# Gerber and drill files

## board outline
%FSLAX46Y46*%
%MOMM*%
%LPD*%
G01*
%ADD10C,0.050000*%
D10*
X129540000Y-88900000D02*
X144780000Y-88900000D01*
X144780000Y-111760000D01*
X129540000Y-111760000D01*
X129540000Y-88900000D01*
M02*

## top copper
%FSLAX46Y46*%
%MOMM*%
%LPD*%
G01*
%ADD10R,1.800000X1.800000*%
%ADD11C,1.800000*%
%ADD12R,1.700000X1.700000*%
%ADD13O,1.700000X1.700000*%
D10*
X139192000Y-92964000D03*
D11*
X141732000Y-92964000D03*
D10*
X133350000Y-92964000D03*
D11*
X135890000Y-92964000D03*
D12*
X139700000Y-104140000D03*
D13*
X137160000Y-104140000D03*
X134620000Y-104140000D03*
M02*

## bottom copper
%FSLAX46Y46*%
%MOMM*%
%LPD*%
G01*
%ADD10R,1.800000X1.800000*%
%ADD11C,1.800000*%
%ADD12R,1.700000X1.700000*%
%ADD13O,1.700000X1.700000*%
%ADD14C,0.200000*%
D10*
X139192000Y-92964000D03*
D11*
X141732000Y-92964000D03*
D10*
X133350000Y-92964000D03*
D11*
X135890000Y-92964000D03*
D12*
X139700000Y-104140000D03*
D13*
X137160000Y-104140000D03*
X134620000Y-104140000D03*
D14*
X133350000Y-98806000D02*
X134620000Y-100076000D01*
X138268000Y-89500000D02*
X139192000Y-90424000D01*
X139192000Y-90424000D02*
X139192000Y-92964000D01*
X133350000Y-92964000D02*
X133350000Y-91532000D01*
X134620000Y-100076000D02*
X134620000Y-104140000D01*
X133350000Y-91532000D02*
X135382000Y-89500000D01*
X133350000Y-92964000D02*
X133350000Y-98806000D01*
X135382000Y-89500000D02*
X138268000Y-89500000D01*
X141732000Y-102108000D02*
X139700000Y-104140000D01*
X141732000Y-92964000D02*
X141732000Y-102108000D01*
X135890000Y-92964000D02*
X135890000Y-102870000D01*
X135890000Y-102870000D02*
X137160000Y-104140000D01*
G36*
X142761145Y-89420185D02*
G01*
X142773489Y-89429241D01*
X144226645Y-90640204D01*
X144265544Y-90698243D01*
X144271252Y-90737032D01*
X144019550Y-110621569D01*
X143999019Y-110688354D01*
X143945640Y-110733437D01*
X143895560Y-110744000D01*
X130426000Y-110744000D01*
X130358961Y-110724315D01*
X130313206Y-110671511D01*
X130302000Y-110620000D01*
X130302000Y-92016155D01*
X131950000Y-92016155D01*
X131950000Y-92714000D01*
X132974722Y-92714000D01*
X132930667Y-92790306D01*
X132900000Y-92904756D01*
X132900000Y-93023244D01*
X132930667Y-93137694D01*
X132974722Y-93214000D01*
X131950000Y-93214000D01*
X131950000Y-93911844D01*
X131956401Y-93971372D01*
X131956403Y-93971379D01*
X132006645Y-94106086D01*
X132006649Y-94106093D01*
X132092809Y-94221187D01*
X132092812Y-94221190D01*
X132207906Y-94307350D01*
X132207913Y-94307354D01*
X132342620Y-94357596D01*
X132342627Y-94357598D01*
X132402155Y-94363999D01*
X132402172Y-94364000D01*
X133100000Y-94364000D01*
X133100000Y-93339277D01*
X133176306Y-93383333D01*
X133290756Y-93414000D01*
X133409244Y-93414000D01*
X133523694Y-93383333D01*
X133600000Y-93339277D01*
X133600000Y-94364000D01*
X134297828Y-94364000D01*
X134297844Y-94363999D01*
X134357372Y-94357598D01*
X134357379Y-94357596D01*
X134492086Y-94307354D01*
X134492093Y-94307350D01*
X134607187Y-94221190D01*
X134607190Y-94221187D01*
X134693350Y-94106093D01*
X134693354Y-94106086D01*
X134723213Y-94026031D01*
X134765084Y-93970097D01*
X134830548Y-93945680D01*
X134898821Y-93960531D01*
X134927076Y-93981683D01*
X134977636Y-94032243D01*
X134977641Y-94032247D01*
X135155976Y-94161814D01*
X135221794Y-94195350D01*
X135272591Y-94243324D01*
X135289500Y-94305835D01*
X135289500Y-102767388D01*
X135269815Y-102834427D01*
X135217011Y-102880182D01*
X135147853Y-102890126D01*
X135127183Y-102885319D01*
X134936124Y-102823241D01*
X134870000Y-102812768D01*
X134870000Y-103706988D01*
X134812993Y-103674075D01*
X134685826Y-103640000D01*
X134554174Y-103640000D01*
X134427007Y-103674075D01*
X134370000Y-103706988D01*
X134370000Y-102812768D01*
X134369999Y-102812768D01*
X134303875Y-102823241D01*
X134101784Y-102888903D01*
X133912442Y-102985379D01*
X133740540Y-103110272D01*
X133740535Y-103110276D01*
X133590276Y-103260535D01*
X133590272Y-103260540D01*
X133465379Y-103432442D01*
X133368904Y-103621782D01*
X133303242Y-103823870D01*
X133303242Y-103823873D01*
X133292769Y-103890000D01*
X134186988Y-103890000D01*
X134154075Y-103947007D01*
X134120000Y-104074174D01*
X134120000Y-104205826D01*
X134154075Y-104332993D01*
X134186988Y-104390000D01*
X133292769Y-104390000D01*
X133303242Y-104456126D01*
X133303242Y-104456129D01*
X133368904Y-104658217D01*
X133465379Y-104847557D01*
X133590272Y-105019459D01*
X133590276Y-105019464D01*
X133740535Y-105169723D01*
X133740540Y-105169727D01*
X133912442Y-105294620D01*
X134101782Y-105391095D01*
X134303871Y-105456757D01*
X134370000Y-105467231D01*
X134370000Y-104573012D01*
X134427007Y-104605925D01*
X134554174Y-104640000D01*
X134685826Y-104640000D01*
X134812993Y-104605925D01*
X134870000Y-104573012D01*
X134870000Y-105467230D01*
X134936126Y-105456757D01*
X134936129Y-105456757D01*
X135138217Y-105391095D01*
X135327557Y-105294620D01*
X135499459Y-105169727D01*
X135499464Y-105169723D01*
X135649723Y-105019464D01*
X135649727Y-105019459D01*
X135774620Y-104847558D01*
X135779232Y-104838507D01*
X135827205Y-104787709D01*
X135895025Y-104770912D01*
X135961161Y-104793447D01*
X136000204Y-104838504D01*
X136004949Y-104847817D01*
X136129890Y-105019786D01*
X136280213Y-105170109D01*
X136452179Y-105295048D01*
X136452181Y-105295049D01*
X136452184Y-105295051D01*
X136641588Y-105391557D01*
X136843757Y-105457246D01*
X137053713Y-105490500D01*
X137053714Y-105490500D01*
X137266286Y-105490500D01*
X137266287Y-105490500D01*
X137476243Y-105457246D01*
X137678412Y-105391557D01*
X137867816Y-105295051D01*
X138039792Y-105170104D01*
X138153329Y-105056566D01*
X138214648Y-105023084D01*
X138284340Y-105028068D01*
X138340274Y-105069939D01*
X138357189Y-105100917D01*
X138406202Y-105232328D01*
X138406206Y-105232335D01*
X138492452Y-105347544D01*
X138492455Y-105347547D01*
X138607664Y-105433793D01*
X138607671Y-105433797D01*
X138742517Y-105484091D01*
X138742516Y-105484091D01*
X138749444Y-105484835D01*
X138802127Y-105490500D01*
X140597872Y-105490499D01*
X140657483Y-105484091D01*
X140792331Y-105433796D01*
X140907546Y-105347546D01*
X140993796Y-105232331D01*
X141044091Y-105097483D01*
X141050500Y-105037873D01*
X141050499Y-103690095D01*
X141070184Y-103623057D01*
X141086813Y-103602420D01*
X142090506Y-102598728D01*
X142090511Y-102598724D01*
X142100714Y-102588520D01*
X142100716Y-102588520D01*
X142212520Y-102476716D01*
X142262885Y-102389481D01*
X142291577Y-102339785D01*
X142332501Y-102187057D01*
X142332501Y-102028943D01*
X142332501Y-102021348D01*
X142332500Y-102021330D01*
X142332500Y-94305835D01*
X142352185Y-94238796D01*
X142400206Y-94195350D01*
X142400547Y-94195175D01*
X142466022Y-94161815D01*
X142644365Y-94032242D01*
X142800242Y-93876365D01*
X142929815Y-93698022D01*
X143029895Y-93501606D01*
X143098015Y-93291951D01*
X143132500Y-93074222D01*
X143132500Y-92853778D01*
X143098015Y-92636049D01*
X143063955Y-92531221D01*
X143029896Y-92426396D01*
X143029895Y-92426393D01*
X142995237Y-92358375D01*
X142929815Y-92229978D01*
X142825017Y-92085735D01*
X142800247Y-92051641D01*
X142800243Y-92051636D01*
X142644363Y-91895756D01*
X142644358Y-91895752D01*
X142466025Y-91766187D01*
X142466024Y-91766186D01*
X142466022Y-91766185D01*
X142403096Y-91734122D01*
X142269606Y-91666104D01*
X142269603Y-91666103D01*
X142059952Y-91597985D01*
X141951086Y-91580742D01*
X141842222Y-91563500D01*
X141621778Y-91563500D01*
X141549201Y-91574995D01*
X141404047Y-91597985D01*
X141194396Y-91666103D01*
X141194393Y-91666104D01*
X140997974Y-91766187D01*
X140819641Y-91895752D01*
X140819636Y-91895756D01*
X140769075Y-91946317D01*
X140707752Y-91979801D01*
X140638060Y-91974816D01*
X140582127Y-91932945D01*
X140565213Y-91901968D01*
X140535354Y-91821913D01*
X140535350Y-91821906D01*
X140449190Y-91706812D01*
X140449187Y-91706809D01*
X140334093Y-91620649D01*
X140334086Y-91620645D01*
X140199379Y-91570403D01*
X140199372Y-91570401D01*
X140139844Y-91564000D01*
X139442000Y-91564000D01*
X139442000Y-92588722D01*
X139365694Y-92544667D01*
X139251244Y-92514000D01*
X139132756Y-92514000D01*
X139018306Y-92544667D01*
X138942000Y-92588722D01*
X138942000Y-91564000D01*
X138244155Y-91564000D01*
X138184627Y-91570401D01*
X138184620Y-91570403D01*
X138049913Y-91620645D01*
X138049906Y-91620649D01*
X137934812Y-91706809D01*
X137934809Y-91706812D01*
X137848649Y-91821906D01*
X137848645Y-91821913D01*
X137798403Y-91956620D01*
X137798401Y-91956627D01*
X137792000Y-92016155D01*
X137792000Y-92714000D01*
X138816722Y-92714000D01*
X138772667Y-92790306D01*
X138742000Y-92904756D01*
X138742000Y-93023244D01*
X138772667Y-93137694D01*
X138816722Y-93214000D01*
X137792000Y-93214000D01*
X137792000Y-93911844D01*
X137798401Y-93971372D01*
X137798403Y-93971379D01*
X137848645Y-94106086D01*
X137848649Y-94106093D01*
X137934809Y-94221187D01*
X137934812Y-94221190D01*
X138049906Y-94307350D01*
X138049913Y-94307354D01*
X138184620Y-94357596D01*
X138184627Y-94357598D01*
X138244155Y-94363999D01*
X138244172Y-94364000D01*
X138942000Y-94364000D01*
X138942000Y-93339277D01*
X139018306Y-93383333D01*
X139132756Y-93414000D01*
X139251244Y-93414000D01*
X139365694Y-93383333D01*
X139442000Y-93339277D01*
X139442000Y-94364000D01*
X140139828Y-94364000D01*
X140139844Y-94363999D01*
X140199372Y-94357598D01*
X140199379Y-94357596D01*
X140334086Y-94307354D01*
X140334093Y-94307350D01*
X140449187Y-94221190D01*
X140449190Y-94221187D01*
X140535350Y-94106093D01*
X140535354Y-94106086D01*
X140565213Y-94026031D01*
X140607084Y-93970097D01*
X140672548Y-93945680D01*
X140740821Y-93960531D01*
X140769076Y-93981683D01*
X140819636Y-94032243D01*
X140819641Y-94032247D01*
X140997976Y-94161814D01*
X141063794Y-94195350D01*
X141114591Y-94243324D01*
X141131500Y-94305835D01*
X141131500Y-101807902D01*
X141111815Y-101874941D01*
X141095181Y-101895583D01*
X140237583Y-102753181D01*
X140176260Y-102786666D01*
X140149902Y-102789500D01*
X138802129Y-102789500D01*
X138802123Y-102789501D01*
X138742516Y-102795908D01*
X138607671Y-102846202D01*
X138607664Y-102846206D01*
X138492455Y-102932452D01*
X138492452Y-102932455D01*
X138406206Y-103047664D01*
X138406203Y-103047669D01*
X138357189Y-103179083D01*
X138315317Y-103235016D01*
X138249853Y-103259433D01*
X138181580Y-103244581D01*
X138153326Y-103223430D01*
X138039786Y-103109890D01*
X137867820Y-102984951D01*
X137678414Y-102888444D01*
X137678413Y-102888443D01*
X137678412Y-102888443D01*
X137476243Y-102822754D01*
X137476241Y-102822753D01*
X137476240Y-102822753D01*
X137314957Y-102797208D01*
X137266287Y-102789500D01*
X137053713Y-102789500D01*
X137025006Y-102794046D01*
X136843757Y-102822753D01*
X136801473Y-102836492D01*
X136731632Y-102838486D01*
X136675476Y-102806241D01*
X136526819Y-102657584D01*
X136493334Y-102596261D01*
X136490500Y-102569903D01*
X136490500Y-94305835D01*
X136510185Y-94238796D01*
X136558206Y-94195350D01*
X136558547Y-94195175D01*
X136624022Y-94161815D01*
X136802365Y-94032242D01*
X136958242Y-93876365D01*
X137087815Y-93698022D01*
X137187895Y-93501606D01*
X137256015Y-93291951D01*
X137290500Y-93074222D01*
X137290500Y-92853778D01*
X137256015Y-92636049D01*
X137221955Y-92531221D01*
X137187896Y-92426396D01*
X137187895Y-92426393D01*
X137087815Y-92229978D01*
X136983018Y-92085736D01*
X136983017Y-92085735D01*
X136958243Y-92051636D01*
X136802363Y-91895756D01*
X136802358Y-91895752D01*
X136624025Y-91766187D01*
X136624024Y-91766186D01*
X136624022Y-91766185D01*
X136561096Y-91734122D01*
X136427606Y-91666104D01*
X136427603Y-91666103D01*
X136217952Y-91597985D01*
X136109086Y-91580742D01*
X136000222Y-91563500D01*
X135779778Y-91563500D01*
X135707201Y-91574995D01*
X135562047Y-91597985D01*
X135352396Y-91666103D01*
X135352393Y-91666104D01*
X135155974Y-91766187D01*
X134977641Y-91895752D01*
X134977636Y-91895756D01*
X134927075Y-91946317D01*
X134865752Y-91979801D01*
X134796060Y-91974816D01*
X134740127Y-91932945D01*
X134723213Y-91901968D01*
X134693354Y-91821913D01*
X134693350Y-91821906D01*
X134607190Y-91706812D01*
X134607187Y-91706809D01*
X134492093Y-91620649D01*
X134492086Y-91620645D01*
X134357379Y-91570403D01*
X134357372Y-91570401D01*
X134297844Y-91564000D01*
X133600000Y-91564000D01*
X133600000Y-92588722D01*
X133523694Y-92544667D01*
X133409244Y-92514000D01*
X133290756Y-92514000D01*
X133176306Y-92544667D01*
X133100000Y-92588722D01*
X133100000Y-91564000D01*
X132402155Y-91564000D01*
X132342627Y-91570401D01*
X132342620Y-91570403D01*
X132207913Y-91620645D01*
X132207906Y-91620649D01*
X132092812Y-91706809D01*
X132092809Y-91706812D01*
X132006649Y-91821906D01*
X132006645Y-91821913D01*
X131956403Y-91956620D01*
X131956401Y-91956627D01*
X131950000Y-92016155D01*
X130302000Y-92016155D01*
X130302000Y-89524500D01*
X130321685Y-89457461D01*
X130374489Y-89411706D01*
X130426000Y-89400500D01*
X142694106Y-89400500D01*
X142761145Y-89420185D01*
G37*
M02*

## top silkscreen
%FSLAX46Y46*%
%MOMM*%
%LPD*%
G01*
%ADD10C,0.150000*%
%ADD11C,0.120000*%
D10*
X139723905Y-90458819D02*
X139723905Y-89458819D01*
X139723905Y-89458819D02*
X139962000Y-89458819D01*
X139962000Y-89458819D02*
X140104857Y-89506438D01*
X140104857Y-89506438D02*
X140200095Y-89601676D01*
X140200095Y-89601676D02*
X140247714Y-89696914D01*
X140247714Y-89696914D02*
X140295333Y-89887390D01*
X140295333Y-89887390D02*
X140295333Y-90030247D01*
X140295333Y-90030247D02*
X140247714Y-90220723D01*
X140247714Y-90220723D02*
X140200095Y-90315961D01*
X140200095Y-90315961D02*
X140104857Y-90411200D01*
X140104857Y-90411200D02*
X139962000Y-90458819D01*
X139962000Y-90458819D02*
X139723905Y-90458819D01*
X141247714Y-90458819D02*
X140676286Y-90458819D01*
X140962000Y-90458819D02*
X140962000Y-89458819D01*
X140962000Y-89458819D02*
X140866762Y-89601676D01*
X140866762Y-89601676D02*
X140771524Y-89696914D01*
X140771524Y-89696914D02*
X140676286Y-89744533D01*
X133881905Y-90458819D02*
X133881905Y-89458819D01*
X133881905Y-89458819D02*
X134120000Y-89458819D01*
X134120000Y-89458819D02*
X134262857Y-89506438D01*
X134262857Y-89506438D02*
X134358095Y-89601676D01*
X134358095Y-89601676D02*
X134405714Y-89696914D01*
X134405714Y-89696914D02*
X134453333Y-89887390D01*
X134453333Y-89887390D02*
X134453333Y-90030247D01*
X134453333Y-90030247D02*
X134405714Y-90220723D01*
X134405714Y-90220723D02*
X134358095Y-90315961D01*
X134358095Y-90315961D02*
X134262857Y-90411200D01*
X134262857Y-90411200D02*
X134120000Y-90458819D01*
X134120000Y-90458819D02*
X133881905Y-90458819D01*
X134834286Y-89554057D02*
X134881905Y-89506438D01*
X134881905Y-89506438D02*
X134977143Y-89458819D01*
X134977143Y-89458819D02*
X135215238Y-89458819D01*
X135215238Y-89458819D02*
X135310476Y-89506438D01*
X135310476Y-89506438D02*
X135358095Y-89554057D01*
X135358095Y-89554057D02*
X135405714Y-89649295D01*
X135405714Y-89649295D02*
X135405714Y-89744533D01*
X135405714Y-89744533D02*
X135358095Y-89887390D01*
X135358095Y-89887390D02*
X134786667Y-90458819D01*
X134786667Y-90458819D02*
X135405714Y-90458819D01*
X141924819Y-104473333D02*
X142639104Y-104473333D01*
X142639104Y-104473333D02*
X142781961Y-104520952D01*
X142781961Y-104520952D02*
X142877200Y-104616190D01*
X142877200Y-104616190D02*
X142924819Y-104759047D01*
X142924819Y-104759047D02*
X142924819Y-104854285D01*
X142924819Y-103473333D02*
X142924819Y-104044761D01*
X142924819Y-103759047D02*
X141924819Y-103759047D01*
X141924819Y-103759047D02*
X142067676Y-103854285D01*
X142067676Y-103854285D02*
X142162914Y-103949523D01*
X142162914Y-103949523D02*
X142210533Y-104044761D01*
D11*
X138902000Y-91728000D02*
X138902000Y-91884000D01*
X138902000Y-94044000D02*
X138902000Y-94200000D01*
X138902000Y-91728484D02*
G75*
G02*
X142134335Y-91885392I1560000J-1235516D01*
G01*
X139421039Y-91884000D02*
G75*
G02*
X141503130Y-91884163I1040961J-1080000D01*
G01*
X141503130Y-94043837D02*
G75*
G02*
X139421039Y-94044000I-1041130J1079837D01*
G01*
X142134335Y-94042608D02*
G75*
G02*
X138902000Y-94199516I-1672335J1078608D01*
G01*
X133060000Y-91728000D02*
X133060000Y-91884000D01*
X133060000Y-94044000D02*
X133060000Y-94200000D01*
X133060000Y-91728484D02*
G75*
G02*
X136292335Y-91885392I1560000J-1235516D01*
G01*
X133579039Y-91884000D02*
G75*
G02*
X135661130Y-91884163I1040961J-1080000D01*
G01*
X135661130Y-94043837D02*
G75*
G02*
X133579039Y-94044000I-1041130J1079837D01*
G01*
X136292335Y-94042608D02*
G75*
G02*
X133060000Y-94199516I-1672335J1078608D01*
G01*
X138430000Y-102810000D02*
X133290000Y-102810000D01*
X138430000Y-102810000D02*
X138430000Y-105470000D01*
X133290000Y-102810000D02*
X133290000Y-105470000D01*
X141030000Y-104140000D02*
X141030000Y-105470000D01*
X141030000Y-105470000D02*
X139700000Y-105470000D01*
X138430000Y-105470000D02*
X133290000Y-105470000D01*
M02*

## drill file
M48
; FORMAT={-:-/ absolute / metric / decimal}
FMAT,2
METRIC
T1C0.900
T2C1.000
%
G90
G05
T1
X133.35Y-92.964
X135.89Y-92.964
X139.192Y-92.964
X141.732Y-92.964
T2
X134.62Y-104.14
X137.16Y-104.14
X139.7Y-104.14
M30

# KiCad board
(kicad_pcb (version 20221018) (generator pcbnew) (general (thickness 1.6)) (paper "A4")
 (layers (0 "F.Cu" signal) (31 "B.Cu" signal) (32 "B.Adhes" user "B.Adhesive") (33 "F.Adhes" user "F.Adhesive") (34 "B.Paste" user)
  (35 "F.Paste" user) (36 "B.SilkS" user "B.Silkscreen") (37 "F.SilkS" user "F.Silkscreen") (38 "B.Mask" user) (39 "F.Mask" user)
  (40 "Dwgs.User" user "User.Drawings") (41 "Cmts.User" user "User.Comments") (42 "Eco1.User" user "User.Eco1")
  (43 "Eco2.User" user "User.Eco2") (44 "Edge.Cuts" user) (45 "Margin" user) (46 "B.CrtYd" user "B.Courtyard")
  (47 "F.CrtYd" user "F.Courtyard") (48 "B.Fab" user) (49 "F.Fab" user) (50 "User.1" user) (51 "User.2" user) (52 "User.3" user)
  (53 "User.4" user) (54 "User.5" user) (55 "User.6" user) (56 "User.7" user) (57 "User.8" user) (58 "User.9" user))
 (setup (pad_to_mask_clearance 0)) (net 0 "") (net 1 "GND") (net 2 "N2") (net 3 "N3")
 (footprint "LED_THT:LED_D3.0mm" (layer "F.Cu") (at 139.192 92.964)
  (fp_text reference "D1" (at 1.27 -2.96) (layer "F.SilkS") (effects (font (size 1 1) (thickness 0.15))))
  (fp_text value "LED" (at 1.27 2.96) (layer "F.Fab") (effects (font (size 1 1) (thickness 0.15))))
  (fp_line (start -0.29 -1.236) (end -0.29 -1.08) (stroke (width 0.12) (type solid)) (layer "F.SilkS"))
  (fp_line (start -0.29 1.08) (end -0.29 1.236) (stroke (width 0.12) (type solid)) (layer "F.SilkS"))
  (fp_arc (start -0.29 -1.235516) (mid 1.366487 -1.987659) (end 2.942335 -1.078608) (stroke (width 0.12) (type solid)) (layer "F.SilkS"))
  (fp_arc (start 0.229039 -1.08) (mid 1.270117 -1.5) (end 2.31113 -1.079837) (stroke (width 0.12) (type solid)) (layer "F.SilkS"))
  (fp_arc (start 2.31113 1.079837) (mid 1.270117 1.5) (end 0.229039 1.08) (stroke (width 0.12) (type solid)) (layer "F.SilkS"))
  (fp_arc (start 2.942335 1.078608) (mid 1.366487 1.987659) (end -0.29 1.235516) (stroke (width 0.12) (type solid)) (layer "F.SilkS"))
  (pad "1" thru_hole rect (at 0 0) (size 1.8 1.8) (drill 0.9) (layers "*.Cu" "*.Mask") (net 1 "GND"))
  (pad "2" thru_hole circle (at 2.54 0) (size 1.8 1.8) (drill 0.9) (layers "*.Cu" "*.Mask") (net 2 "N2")))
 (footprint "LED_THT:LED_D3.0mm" (layer "F.Cu") (at 133.35 92.964)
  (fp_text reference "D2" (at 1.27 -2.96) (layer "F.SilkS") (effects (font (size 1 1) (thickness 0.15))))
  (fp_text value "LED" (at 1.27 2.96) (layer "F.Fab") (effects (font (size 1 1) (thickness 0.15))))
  (fp_line (start -0.29 -1.236) (end -0.29 -1.08) (stroke (width 0.12) (type solid)) (layer "F.SilkS"))
  (fp_line (start -0.29 1.08) (end -0.29 1.236) (stroke (width 0.12) (type solid)) (layer "F.SilkS"))
  (fp_arc (start -0.29 -1.235516) (mid 1.366487 -1.987659) (end 2.942335 -1.078608) (stroke (width 0.12) (type solid)) (layer "F.SilkS"))
  (fp_arc (start 0.229039 -1.08) (mid 1.270117 -1.5) (end 2.31113 -1.079837) (stroke (width 0.12) (type solid)) (layer "F.SilkS"))
  (fp_arc (start 2.31113 1.079837) (mid 1.270117 1.5) (end 0.229039 1.08) (stroke (width 0.12) (type solid)) (layer "F.SilkS"))
  (fp_arc (start 2.942335 1.078608) (mid 1.366487 1.987659) (end -0.29 1.235516) (stroke (width 0.12) (type solid)) (layer "F.SilkS"))
  (pad "1" thru_hole rect (at 0 0) (size 1.8 1.8) (drill 0.9) (layers "*.Cu" "*.Mask") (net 1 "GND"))
  (pad "2" thru_hole circle (at 2.54 0) (size 1.8 1.8) (drill 0.9) (layers "*.Cu" "*.Mask") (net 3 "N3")))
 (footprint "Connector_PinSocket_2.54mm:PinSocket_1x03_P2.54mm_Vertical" (layer "F.Cu") (at 139.7 104.14 -90)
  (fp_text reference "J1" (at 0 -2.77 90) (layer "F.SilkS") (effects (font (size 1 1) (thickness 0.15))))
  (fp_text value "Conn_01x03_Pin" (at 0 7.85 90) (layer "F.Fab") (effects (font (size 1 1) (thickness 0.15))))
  (fp_line (start -1.33 1.27) (end -1.33 6.41) (stroke (width 0.12) (type solid)) (layer "F.SilkS"))
  (fp_line (start -1.33 1.27) (end 1.33 1.27) (stroke (width 0.12) (type solid)) (layer "F.SilkS"))
  (fp_line (start -1.33 6.41) (end 1.33 6.41) (stroke (width 0.12) (type solid)) (layer "F.SilkS"))
  (fp_line (start 0 -1.33) (end 1.33 -1.33) (stroke (width 0.12) (type solid)) (layer "F.SilkS"))
  (fp_line (start 1.33 -1.33) (end 1.33 0) (stroke (width 0.12) (type solid)) (layer "F.SilkS"))
  (fp_line (start 1.33 1.27) (end 1.33 6.41) (stroke (width 0.12) (type solid)) (layer "F.SilkS"))
  (pad "1" thru_hole rect (at 0 0 270) (size 1.7 1.7) (drill 1) (layers "*.Cu" "*.Mask") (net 2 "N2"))
  (pad "2" thru_hole oval (at 0 2.54 270) (size 1.7 1.7) (drill 1) (layers "*.Cu" "*.Mask") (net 3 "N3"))
  (pad "3" thru_hole oval (at 0 5.08 270) (size 1.7 1.7) (drill 1) (layers "*.Cu" "*.Mask") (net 1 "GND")))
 (gr_rect (start 129.54 88.9) (end 144.78 111.76) (stroke (width 0.05) (type default)) (fill none) (layer "Edge.Cuts"))
 (segment (start 133.35 98.806) (end 134.62 100.076) (width 0.2) (layer "B.Cu") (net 1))
 (segment (start 138.268 89.5) (end 139.192 90.424) (width 0.2) (layer "B.Cu") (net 1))
 (segment (start 139.192 90.424) (end 139.192 92.964) (width 0.2) (layer "B.Cu") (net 1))
 (segment (start 133.35 92.964) (end 133.35 91.532) (width 0.2) (layer "B.Cu") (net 1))
 (segment (start 134.62 100.076) (end 134.62 104.14) (width 0.2) (layer "B.Cu") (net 1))
 (segment (start 133.35 91.532) (end 135.382 89.5) (width 0.2) (layer "B.Cu") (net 1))
 (segment (start 133.35 92.964) (end 133.35 98.806) (width 0.2) (layer "B.Cu") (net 1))
 (segment (start 135.382 89.5) (end 138.268 89.5) (width 0.2) (layer "B.Cu") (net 1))
 (segment (start 141.732 102.108) (end 139.7 104.14) (width 0.2) (layer "B.Cu") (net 2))
 (segment (start 141.732 92.964) (end 141.732 102.108) (width 0.2) (layer "B.Cu") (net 2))
 (segment (start 135.89 92.964) (end 135.89 102.87) (width 0.2) (layer "B.Cu") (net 3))
 (segment (start 135.89 102.87) (end 137.16 104.14) (width 0.2) (layer "B.Cu") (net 3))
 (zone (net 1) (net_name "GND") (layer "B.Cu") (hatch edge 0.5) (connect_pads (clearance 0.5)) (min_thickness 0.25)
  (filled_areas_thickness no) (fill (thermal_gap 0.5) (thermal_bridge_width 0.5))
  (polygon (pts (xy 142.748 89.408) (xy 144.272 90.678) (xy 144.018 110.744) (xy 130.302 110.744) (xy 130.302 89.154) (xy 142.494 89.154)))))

